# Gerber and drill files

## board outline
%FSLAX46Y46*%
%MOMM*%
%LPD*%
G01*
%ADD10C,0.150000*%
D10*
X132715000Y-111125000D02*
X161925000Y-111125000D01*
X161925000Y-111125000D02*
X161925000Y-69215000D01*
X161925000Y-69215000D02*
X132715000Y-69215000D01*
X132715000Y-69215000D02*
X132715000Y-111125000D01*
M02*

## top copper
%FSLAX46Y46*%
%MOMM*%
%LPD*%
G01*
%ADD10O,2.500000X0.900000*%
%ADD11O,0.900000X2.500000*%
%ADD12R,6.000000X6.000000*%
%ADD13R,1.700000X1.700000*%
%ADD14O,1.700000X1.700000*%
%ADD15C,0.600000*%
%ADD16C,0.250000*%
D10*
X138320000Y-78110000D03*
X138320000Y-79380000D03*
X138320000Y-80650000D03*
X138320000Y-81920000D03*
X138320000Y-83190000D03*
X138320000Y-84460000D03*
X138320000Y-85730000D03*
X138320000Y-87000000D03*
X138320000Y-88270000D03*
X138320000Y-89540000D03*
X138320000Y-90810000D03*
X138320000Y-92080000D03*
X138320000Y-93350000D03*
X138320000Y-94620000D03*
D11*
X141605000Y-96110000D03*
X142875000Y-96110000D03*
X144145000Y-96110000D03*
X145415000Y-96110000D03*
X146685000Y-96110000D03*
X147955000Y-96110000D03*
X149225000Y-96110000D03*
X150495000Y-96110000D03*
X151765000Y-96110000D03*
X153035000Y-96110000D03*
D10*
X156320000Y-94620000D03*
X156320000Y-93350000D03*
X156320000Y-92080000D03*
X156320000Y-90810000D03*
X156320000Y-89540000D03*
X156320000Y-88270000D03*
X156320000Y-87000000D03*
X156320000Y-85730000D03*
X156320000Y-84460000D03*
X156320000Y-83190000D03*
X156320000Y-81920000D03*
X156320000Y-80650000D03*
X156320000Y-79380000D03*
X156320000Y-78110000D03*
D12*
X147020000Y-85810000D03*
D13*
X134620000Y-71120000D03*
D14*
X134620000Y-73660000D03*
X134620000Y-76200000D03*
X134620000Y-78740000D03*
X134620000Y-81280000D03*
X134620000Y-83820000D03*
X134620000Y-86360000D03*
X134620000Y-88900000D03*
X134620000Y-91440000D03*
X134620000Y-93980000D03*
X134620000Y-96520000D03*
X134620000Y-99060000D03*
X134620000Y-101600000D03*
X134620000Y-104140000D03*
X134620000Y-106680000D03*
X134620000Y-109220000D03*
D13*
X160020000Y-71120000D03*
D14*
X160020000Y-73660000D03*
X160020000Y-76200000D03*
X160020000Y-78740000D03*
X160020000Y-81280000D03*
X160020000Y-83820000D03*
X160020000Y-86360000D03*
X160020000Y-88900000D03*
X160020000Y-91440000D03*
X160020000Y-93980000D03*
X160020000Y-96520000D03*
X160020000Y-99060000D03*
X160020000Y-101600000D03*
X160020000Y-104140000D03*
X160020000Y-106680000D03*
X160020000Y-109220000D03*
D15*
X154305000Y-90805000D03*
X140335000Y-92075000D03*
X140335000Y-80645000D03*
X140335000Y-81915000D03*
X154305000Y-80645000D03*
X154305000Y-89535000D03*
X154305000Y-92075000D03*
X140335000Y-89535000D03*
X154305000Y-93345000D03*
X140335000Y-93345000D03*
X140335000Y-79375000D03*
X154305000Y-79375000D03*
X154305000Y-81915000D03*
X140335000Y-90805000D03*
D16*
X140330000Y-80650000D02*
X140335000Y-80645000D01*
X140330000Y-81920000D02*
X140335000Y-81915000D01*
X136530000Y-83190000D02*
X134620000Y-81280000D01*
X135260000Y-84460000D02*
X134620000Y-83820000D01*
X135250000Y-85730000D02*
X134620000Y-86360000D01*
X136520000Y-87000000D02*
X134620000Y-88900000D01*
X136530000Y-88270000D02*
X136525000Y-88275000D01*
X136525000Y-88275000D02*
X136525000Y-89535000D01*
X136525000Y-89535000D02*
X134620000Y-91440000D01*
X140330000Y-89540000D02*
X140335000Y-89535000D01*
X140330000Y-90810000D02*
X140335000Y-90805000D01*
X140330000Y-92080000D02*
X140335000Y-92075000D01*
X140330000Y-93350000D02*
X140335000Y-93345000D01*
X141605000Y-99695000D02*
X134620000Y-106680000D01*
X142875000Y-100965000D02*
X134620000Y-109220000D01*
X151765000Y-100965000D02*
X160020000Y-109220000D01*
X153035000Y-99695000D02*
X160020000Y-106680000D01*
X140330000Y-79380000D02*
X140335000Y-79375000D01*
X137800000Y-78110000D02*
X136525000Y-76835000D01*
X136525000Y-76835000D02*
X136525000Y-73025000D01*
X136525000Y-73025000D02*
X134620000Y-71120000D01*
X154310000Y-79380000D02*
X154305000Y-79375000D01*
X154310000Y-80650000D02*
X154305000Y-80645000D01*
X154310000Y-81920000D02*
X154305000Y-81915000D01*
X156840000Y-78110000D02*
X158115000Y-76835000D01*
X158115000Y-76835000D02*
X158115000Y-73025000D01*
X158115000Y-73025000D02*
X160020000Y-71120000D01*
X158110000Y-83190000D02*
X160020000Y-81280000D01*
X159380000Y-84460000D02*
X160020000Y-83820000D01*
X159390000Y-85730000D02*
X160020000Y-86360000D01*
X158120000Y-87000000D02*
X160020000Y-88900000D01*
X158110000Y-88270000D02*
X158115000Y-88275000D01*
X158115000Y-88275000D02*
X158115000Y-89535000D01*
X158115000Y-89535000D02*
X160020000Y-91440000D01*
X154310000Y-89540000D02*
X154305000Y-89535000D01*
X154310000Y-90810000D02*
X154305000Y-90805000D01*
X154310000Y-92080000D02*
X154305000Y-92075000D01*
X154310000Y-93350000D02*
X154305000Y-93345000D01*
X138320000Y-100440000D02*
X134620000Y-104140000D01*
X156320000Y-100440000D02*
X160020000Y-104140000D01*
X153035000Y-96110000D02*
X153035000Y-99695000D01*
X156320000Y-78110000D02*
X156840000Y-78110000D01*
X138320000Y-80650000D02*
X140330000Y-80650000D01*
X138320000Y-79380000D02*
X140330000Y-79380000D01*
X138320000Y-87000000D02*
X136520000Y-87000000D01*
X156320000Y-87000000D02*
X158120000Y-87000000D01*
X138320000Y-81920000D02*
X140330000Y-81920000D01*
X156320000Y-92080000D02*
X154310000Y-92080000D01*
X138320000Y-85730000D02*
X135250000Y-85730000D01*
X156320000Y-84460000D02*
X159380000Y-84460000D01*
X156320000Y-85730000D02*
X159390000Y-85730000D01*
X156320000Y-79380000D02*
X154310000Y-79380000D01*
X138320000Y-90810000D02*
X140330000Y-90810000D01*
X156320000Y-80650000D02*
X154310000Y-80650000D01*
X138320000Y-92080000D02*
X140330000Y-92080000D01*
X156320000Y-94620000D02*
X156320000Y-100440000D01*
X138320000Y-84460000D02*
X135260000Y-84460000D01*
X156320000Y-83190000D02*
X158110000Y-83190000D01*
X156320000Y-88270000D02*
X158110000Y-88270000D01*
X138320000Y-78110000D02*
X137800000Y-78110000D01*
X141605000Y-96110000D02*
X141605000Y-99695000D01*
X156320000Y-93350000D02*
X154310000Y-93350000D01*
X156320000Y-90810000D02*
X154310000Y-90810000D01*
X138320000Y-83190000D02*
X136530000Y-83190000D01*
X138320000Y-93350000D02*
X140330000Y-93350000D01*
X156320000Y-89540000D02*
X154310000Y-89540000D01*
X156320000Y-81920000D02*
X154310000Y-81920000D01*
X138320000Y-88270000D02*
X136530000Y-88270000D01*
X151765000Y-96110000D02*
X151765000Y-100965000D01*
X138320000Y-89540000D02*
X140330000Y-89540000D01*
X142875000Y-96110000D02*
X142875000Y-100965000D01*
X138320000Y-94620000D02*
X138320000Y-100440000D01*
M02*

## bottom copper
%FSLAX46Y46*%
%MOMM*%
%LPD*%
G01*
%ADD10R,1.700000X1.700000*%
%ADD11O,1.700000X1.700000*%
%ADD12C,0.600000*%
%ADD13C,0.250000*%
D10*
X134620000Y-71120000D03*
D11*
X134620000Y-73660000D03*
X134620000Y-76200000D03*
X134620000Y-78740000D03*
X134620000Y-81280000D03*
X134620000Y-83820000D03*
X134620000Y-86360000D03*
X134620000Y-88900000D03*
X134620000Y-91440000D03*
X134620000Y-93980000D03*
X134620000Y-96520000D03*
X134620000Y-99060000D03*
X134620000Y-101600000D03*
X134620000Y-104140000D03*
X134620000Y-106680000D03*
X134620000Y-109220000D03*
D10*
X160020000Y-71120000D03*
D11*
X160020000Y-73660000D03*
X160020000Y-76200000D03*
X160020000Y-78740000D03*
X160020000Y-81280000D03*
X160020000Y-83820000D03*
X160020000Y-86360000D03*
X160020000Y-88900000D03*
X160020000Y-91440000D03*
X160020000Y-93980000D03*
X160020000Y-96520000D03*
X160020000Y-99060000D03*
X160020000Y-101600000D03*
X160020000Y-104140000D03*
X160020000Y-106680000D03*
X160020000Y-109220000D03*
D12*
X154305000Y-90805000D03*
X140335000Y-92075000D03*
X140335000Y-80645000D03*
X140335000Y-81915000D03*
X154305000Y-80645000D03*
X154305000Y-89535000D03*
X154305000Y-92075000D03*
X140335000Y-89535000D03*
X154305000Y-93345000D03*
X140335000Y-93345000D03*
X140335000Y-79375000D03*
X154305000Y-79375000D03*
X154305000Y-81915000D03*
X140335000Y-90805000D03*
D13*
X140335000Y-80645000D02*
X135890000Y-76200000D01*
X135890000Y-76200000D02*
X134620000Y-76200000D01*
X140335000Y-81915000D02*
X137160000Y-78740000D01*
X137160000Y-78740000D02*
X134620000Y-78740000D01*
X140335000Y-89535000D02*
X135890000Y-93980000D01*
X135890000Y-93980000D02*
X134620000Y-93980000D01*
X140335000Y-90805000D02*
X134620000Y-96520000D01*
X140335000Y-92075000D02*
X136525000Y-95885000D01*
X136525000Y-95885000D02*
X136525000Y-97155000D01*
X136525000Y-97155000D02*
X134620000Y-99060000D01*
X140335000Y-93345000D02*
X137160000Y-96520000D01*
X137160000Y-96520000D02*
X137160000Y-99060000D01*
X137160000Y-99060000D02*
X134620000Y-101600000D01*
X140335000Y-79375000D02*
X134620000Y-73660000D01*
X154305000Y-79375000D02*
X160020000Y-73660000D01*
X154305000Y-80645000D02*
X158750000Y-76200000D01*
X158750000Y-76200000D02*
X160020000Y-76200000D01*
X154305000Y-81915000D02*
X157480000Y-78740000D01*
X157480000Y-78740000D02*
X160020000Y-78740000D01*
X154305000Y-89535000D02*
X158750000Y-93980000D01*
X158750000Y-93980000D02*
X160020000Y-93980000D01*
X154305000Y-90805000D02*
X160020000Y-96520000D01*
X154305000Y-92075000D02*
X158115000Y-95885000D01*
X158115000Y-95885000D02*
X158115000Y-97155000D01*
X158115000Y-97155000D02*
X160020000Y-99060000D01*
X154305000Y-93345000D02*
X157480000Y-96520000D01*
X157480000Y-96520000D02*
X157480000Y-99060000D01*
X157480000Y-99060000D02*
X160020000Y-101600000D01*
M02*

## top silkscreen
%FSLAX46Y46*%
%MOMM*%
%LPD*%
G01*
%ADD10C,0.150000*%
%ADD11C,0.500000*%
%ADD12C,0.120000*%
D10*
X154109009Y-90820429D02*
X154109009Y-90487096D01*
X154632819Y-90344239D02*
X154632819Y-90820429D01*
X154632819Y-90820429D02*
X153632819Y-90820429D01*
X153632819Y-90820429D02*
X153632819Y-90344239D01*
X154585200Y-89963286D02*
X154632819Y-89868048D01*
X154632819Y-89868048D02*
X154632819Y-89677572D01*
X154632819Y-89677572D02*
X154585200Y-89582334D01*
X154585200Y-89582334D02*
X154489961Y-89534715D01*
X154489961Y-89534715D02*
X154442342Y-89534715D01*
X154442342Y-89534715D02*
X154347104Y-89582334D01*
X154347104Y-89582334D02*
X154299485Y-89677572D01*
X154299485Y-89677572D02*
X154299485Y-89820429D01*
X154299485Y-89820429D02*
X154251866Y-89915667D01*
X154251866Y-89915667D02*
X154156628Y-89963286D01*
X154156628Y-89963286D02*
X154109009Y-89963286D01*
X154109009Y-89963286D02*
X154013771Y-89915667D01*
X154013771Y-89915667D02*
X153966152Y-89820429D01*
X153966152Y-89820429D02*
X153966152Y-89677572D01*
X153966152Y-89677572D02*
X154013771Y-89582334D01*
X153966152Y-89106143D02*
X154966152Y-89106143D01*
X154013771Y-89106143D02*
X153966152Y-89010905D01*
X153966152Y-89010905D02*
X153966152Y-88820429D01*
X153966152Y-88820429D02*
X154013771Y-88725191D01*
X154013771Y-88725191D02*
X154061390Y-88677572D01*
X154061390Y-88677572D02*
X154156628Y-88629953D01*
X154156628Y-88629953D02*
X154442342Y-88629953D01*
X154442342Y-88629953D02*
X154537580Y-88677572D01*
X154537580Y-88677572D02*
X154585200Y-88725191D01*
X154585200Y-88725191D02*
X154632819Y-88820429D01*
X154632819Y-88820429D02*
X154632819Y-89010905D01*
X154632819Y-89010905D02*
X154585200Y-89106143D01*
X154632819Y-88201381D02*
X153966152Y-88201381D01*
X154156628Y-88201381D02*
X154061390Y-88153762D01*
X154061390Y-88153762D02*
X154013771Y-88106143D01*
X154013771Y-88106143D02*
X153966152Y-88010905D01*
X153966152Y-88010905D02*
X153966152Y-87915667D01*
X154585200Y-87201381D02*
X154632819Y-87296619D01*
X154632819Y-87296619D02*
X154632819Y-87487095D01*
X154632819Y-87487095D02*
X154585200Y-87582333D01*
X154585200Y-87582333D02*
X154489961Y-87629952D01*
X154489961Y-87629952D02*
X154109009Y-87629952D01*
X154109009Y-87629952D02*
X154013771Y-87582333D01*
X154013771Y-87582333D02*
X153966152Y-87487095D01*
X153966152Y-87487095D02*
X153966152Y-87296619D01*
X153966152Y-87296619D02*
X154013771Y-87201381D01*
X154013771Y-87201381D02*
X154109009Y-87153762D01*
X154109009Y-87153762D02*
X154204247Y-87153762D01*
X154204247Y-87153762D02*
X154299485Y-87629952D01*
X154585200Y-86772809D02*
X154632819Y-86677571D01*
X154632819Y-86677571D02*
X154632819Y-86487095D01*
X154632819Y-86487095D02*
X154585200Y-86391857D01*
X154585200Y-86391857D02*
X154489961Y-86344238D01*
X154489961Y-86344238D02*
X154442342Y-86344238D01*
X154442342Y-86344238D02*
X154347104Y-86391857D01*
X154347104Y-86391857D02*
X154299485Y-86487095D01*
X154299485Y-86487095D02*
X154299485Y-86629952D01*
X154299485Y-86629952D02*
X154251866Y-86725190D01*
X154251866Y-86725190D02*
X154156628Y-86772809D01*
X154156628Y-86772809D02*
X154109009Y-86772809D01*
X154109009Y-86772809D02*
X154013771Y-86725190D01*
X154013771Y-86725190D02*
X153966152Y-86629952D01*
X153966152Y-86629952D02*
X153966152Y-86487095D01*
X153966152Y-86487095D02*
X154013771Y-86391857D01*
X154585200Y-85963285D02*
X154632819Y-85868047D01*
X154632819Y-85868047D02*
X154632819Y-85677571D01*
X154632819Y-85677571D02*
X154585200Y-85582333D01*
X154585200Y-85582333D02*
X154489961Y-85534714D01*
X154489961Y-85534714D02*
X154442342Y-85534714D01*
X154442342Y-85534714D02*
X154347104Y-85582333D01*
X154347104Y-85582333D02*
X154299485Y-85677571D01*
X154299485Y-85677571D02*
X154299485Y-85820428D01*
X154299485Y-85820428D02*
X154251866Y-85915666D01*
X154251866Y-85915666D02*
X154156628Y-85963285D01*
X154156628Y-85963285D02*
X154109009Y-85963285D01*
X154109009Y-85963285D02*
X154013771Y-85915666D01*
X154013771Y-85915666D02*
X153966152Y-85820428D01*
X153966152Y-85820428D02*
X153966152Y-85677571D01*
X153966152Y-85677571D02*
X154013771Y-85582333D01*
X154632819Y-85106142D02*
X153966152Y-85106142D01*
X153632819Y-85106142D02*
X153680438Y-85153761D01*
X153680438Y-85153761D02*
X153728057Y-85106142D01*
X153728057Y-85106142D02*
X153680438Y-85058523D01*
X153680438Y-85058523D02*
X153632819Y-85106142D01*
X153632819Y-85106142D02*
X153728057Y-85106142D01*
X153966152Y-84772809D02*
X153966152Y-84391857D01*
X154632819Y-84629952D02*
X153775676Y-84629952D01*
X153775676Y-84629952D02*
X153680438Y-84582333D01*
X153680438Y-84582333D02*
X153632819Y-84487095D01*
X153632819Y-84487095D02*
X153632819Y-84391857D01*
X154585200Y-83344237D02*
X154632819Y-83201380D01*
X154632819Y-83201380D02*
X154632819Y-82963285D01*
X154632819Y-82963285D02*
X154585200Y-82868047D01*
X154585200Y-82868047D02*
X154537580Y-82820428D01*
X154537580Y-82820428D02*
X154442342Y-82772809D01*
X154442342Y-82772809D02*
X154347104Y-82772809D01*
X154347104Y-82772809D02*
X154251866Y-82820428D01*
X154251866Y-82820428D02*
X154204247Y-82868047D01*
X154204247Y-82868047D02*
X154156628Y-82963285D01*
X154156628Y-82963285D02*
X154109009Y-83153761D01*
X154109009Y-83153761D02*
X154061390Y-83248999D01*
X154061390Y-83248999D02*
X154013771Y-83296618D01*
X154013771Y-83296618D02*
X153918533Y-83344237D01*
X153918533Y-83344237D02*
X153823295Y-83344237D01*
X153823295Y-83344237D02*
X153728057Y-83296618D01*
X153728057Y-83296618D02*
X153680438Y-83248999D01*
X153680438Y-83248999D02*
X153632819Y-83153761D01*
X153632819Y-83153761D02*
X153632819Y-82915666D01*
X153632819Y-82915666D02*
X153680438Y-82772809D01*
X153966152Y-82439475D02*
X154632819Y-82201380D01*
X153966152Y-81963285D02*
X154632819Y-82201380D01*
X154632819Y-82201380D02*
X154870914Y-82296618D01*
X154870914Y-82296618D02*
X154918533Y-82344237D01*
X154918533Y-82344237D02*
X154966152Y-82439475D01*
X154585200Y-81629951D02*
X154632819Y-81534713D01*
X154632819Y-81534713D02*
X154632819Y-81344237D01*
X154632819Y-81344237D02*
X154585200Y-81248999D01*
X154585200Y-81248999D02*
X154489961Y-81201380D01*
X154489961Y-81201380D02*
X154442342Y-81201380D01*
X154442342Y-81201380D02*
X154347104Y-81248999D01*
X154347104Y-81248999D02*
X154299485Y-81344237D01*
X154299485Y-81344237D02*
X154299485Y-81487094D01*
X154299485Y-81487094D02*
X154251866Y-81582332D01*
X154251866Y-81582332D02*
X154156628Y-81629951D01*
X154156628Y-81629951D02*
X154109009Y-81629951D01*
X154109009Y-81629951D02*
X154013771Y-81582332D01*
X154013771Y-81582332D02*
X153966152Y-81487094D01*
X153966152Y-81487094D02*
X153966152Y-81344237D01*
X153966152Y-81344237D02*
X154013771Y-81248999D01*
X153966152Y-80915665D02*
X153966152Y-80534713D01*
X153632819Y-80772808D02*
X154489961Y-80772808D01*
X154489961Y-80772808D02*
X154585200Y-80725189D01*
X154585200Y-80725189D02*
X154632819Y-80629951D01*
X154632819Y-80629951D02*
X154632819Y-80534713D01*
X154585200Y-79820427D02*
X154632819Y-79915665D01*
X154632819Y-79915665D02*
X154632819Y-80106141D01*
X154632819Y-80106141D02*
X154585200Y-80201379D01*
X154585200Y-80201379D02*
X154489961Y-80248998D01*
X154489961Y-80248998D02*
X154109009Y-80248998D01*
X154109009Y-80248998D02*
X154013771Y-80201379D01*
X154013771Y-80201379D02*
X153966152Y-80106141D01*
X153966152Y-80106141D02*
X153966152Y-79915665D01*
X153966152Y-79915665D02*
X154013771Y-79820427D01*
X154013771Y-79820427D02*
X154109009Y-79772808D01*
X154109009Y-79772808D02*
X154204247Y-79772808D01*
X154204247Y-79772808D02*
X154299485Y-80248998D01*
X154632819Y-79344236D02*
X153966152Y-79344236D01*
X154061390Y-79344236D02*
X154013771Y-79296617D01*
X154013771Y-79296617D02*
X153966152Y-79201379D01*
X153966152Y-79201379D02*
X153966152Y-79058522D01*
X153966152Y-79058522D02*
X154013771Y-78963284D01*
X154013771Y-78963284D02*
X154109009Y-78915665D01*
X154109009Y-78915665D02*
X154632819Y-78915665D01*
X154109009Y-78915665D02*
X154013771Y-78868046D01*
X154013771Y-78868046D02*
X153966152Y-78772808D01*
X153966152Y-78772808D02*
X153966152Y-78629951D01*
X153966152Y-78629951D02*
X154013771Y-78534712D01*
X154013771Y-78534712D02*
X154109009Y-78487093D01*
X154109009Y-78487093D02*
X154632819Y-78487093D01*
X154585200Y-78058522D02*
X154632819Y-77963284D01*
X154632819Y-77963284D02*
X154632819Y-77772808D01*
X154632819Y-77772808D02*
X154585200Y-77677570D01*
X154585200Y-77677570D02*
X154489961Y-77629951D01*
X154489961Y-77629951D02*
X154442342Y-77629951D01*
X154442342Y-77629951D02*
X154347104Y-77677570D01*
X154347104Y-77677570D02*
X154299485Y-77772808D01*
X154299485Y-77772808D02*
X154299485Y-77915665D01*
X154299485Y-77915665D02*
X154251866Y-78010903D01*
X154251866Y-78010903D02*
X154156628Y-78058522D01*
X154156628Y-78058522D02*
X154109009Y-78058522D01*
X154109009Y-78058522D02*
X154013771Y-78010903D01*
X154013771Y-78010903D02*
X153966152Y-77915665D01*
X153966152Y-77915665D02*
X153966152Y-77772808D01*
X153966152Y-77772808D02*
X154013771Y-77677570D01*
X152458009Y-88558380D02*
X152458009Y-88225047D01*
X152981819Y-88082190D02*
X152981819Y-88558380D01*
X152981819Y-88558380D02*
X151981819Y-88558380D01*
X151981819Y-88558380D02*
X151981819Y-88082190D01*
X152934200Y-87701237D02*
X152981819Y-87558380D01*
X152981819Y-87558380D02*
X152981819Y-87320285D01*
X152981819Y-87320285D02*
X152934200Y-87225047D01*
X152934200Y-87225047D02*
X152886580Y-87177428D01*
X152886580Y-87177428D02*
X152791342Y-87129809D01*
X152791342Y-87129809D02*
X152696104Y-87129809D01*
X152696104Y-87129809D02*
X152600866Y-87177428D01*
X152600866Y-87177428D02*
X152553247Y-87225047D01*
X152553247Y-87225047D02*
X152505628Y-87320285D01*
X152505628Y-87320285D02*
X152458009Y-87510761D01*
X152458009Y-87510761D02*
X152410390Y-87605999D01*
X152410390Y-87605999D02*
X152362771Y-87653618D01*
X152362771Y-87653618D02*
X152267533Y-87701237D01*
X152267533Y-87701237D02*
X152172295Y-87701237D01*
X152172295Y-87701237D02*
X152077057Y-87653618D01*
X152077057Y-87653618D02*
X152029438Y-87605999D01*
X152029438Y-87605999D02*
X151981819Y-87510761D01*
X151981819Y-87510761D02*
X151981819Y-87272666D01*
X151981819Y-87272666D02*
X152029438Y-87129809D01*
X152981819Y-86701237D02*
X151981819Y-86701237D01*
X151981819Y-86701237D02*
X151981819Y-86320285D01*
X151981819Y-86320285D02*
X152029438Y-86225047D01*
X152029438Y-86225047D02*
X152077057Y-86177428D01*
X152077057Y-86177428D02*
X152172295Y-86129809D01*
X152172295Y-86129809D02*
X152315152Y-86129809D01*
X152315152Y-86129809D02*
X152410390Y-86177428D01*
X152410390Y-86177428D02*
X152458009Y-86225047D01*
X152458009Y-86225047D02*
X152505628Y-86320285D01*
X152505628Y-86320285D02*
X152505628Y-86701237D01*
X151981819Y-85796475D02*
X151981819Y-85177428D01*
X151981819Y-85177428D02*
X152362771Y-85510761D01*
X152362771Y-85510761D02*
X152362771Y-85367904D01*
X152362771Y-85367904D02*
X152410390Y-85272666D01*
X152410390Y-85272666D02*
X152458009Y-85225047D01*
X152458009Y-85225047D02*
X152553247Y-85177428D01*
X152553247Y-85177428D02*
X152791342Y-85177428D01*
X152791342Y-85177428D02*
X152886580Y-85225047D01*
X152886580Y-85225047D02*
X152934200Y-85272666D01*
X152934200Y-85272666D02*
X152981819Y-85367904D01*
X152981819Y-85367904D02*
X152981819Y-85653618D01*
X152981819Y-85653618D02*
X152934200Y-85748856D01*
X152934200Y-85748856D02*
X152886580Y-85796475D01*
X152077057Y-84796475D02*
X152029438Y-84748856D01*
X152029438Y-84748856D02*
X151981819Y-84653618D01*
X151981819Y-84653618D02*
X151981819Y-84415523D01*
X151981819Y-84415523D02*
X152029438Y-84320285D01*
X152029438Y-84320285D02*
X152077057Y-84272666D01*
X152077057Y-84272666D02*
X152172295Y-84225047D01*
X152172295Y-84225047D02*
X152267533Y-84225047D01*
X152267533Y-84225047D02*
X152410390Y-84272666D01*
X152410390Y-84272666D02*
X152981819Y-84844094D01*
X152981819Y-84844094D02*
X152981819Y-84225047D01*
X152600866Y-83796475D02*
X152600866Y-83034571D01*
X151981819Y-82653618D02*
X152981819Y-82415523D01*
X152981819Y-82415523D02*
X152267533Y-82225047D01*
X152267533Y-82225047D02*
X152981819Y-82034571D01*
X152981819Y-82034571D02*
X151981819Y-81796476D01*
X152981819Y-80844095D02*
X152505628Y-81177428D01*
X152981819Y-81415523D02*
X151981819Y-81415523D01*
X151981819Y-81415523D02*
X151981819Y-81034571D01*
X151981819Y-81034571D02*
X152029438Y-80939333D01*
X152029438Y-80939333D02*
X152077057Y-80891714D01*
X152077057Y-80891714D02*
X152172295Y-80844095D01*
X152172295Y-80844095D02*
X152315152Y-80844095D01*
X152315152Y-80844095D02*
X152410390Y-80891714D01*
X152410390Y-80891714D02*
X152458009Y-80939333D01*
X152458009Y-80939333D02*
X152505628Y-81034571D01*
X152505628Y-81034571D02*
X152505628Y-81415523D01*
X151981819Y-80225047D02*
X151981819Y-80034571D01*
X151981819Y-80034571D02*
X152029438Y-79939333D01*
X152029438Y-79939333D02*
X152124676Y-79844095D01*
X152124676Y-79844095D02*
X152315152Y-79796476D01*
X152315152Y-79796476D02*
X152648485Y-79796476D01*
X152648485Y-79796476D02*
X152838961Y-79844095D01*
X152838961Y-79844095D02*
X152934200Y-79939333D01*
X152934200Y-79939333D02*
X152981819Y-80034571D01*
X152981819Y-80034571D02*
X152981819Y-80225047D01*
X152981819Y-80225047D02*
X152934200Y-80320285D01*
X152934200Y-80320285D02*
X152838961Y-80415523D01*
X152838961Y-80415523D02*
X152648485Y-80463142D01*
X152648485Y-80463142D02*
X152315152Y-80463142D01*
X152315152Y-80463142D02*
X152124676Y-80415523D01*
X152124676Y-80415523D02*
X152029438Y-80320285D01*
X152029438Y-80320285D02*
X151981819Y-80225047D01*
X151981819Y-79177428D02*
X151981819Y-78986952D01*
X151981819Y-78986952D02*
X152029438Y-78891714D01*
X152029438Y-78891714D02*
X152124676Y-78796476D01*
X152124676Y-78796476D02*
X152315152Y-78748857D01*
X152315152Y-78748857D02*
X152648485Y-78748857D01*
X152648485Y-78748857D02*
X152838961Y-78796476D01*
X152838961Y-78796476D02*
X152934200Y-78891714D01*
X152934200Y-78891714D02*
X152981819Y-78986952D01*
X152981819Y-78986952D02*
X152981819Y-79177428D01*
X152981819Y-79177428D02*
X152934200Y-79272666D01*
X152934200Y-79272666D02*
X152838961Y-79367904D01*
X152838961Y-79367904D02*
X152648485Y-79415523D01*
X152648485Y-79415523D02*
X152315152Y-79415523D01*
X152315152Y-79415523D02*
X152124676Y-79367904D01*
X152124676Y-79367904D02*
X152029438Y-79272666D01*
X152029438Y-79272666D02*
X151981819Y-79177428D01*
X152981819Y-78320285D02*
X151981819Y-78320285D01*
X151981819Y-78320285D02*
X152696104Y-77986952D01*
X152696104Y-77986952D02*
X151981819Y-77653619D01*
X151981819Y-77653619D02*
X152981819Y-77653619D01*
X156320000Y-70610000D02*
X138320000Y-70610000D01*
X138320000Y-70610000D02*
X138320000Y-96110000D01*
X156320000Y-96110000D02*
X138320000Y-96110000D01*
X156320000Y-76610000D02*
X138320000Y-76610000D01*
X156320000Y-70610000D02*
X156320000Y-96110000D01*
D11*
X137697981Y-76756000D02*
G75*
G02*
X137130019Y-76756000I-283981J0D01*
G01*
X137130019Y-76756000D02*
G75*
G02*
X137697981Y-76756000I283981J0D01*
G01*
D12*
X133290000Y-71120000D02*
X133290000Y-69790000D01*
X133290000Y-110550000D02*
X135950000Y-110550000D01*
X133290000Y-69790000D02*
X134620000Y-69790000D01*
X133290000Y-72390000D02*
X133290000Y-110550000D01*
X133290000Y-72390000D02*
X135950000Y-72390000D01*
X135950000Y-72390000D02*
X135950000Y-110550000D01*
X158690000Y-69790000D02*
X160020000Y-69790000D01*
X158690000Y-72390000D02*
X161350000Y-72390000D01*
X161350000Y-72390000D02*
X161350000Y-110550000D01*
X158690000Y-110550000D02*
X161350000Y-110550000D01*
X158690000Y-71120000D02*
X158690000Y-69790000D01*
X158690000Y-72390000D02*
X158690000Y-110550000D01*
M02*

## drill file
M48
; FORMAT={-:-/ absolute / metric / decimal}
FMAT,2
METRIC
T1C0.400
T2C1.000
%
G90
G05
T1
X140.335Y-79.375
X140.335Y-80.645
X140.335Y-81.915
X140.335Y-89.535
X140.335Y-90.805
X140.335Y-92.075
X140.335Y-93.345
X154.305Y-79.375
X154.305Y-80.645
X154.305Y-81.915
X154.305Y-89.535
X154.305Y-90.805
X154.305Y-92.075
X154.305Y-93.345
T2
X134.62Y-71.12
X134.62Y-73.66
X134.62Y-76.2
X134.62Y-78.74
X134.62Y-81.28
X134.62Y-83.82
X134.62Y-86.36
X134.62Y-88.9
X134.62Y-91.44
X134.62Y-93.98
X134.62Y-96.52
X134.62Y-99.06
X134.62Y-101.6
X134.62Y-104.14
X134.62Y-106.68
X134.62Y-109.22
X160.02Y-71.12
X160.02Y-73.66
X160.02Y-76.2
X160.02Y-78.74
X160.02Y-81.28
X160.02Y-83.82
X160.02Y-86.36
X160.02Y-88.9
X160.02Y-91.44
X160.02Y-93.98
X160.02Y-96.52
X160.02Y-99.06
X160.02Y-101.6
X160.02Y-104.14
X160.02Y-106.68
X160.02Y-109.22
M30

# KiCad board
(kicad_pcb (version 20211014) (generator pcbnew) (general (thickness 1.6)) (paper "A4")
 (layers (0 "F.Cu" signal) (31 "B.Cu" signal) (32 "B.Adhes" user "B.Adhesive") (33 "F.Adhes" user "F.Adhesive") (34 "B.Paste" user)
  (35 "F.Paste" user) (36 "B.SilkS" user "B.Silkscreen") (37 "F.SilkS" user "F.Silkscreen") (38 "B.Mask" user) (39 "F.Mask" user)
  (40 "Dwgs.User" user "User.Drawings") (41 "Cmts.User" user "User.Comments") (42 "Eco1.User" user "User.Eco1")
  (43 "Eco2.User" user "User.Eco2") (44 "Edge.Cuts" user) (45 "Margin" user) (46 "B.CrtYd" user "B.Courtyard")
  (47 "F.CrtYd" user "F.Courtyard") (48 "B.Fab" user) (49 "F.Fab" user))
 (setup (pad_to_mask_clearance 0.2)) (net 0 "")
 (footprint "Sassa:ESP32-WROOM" (layer "F.Cu") (at 147.32 86.36 180)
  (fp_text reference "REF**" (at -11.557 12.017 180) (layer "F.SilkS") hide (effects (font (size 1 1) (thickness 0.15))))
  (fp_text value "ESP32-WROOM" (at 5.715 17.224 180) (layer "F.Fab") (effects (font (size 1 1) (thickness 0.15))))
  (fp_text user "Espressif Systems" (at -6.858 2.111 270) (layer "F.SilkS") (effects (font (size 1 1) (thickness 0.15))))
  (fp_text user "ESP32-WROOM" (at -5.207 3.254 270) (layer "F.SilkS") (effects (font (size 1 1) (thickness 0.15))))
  (fp_line (start -9 15.75) (end 9 15.75) (layer "F.SilkS") (width 0.15))
  (fp_line (start 9 15.75) (end 9 -9.75) (layer "F.SilkS") (width 0.15))
  (fp_line (start -9 -9.75) (end 9 -9.75) (layer "F.SilkS") (width 0.15))
  (fp_line (start -9 9.75) (end 9 9.75) (layer "F.SilkS") (width 0.15))
  (fp_line (start -9 15.75) (end -9 -9.75) (layer "F.SilkS") (width 0.15))
  (fp_circle (center 9.906 9.604) (end 10.033 9.858) (layer "F.SilkS") (width 0.5) (fill none))
  (pad "1" smd oval locked (at 9 8.25 180) (size 2.5 0.9) (layers "F.Cu" "F.Paste" "F.Mask"))
  (pad "2" smd oval locked (at 9 6.98 180) (size 2.5 0.9) (layers "F.Cu" "F.Paste" "F.Mask"))
  (pad "3" smd oval locked (at 9 5.71 180) (size 2.5 0.9) (layers "F.Cu" "F.Paste" "F.Mask"))
  (pad "4" smd oval locked (at 9 4.44 180) (size 2.5 0.9) (layers "F.Cu" "F.Paste" "F.Mask"))
  (pad "5" smd oval locked (at 9 3.17 180) (size 2.5 0.9) (layers "F.Cu" "F.Paste" "F.Mask"))
  (pad "6" smd oval locked (at 9 1.9 180) (size 2.5 0.9) (layers "F.Cu" "F.Paste" "F.Mask"))
  (pad "7" smd oval locked (at 9 0.63 180) (size 2.5 0.9) (layers "F.Cu" "F.Paste" "F.Mask"))
  (pad "8" smd oval locked (at 9 -0.64 180) (size 2.5 0.9) (layers "F.Cu" "F.Paste" "F.Mask"))
  (pad "9" smd oval locked (at 9 -1.91 180) (size 2.5 0.9) (layers "F.Cu" "F.Paste" "F.Mask"))
  (pad "10" smd oval locked (at 9 -3.18 180) (size 2.5 0.9) (layers "F.Cu" "F.Paste" "F.Mask"))
  (pad "11" smd oval locked (at 9 -4.45 180) (size 2.5 0.9) (layers "F.Cu" "F.Paste" "F.Mask"))
  (pad "12" smd oval locked (at 9 -5.72 180) (size 2.5 0.9) (layers "F.Cu" "F.Paste" "F.Mask"))
  (pad "13" smd oval locked (at 9 -6.99 180) (size 2.5 0.9) (layers "F.Cu" "F.Paste" "F.Mask"))
  (pad "14" smd oval locked (at 9 -8.26 180) (size 2.5 0.9) (layers "F.Cu" "F.Paste" "F.Mask"))
  (pad "15" smd oval locked (at 5.715 -9.75 180) (size 0.9 2.5) (layers "F.Cu" "F.Paste" "F.Mask"))
  (pad "16" smd oval locked (at 4.445 -9.75 180) (size 0.9 2.5) (layers "F.Cu" "F.Paste" "F.Mask"))
  (pad "17" smd oval locked (at 3.175 -9.75 180) (size 0.9 2.5) (layers "F.Cu" "F.Paste" "F.Mask"))
  (pad "18" smd oval locked (at 1.905 -9.75 180) (size 0.9 2.5) (layers "F.Cu" "F.Paste" "F.Mask"))
  (pad "19" smd oval locked (at 0.635 -9.75 180) (size 0.9 2.5) (layers "F.Cu" "F.Paste" "F.Mask"))
  (pad "20" smd oval locked (at -0.635 -9.75 180) (size 0.9 2.5) (layers "F.Cu" "F.Paste" "F.Mask"))
  (pad "21" smd oval locked (at -1.905 -9.75 180) (size 0.9 2.5) (layers "F.Cu" "F.Paste" "F.Mask"))
  (pad "22" smd oval locked (at -3.175 -9.75 180) (size 0.9 2.5) (layers "F.Cu" "F.Paste" "F.Mask"))
  (pad "23" smd oval locked (at -4.445 -9.75 180) (size 0.9 2.5) (layers "F.Cu" "F.Paste" "F.Mask"))
  (pad "24" smd oval locked (at -5.715 -9.75 180) (size 0.9 2.5) (layers "F.Cu" "F.Paste" "F.Mask"))
  (pad "25" smd oval locked (at -9 -8.26 180) (size 2.5 0.9) (layers "F.Cu" "F.Paste" "F.Mask"))
  (pad "26" smd oval locked (at -9 -6.99 180) (size 2.5 0.9) (layers "F.Cu" "F.Paste" "F.Mask"))
  (pad "27" smd oval locked (at -9 -5.72 180) (size 2.5 0.9) (layers "F.Cu" "F.Paste" "F.Mask"))
  (pad "28" smd oval locked (at -9 -4.45 180) (size 2.5 0.9) (layers "F.Cu" "F.Paste" "F.Mask"))
  (pad "29" smd oval locked (at -9 -3.18 180) (size 2.5 0.9) (layers "F.Cu" "F.Paste" "F.Mask"))
  (pad "30" smd oval locked (at -9 -1.91 180) (size 2.5 0.9) (layers "F.Cu" "F.Paste" "F.Mask"))
  (pad "31" smd oval locked (at -9 -0.64 180) (size 2.5 0.9) (layers "F.Cu" "F.Paste" "F.Mask"))
  (pad "32" smd oval locked (at -9 0.63 180) (size 2.5 0.9) (layers "F.Cu" "F.Paste" "F.Mask"))
  (pad "33" smd oval locked (at -9 1.9 180) (size 2.5 0.9) (layers "F.Cu" "F.Paste" "F.Mask"))
  (pad "34" smd oval locked (at -9 3.17 180) (size 2.5 0.9) (layers "F.Cu" "F.Paste" "F.Mask"))
  (pad "35" smd oval locked (at -9 4.44 180) (size 2.5 0.9) (layers "F.Cu" "F.Paste" "F.Mask"))
  (pad "36" smd oval locked (at -9 5.71 180) (size 2.5 0.9) (layers "F.Cu" "F.Paste" "F.Mask"))
  (pad "37" smd oval locked (at -9 6.98 180) (size 2.5 0.9) (layers "F.Cu" "F.Paste" "F.Mask"))
  (pad "38" smd oval locked (at -9 8.25 180) (size 2.5 0.9) (layers "F.Cu" "F.Paste" "F.Mask"))
  (pad "39" smd rect locked (at 0.3 0.55 180) (size 6 6) (layers "F.Cu" "F.Paste" "F.Mask")))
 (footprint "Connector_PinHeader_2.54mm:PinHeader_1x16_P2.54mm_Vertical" (layer "F.Cu") (at 134.62 71.12)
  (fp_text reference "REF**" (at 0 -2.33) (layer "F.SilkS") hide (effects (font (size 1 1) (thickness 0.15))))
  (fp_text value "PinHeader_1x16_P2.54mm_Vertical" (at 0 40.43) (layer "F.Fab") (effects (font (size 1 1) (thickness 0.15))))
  (fp_line (start -1.33 0) (end -1.33 -1.33) (layer "F.SilkS") (width 0.12))
  (fp_line (start -1.33 39.43) (end 1.33 39.43) (layer "F.SilkS") (width 0.12))
  (fp_line (start -1.33 -1.33) (end 0 -1.33) (layer "F.SilkS") (width 0.12))
  (fp_line (start -1.33 1.27) (end -1.33 39.43) (layer "F.SilkS") (width 0.12))
  (fp_line (start -1.33 1.27) (end 1.33 1.27) (layer "F.SilkS") (width 0.12))
  (fp_line (start 1.33 1.27) (end 1.33 39.43) (layer "F.SilkS") (width 0.12))
  (pad "1" thru_hole rect (at 0 0) (size 1.7 1.7) (drill 1) (layers *.Cu *.Mask))
  (pad "2" thru_hole oval (at 0 2.54) (size 1.7 1.7) (drill 1) (layers *.Cu *.Mask))
  (pad "3" thru_hole oval (at 0 5.08) (size 1.7 1.7) (drill 1) (layers *.Cu *.Mask))
  (pad "4" thru_hole oval (at 0 7.62) (size 1.7 1.7) (drill 1) (layers *.Cu *.Mask))
  (pad "5" thru_hole oval (at 0 10.16) (size 1.7 1.7) (drill 1) (layers *.Cu *.Mask))
  (pad "6" thru_hole oval (at 0 12.7) (size 1.7 1.7) (drill 1) (layers *.Cu *.Mask))
  (pad "7" thru_hole oval (at 0 15.24) (size 1.7 1.7) (drill 1) (layers *.Cu *.Mask))
  (pad "8" thru_hole oval (at 0 17.78) (size 1.7 1.7) (drill 1) (layers *.Cu *.Mask))
  (pad "9" thru_hole oval (at 0 20.32) (size 1.7 1.7) (drill 1) (layers *.Cu *.Mask))
  (pad "10" thru_hole oval (at 0 22.86) (size 1.7 1.7) (drill 1) (layers *.Cu *.Mask))
  (pad "11" thru_hole oval (at 0 25.4) (size 1.7 1.7) (drill 1) (layers *.Cu *.Mask))
  (pad "12" thru_hole oval (at 0 27.94) (size 1.7 1.7) (drill 1) (layers *.Cu *.Mask))
  (pad "13" thru_hole oval (at 0 30.48) (size 1.7 1.7) (drill 1) (layers *.Cu *.Mask))
  (pad "14" thru_hole oval (at 0 33.02) (size 1.7 1.7) (drill 1) (layers *.Cu *.Mask))
  (pad "15" thru_hole oval (at 0 35.56) (size 1.7 1.7) (drill 1) (layers *.Cu *.Mask))
  (pad "16" thru_hole oval (at 0 38.1) (size 1.7 1.7) (drill 1) (layers *.Cu *.Mask)))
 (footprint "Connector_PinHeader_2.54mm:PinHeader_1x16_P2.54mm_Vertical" (layer "F.Cu") (at 160.02 71.12)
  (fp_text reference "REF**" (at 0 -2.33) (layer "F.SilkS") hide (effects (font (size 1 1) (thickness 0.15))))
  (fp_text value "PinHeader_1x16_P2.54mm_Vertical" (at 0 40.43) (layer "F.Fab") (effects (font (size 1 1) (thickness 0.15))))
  (fp_line (start -1.33 -1.33) (end 0 -1.33) (layer "F.SilkS") (width 0.12))
  (fp_line (start -1.33 1.27) (end 1.33 1.27) (layer "F.SilkS") (width 0.12))
  (fp_line (start 1.33 1.27) (end 1.33 39.43) (layer "F.SilkS") (width 0.12))
  (fp_line (start -1.33 39.43) (end 1.33 39.43) (layer "F.SilkS") (width 0.12))
  (fp_line (start -1.33 0) (end -1.33 -1.33) (layer "F.SilkS") (width 0.12))
  (fp_line (start -1.33 1.27) (end -1.33 39.43) (layer "F.SilkS") (width 0.12))
  (pad "1" thru_hole rect (at 0 0) (size 1.7 1.7) (drill 1) (layers *.Cu *.Mask))
  (pad "2" thru_hole oval (at 0 2.54) (size 1.7 1.7) (drill 1) (layers *.Cu *.Mask))
  (pad "3" thru_hole oval (at 0 5.08) (size 1.7 1.7) (drill 1) (layers *.Cu *.Mask))
  (pad "4" thru_hole oval (at 0 7.62) (size 1.7 1.7) (drill 1) (layers *.Cu *.Mask))
  (pad "5" thru_hole oval (at 0 10.16) (size 1.7 1.7) (drill 1) (layers *.Cu *.Mask))
  (pad "6" thru_hole oval (at 0 12.7) (size 1.7 1.7) (drill 1) (layers *.Cu *.Mask))
  (pad "7" thru_hole oval (at 0 15.24) (size 1.7 1.7) (drill 1) (layers *.Cu *.Mask))
  (pad "8" thru_hole oval (at 0 17.78) (size 1.7 1.7) (drill 1) (layers *.Cu *.Mask))
  (pad "9" thru_hole oval (at 0 20.32) (size 1.7 1.7) (drill 1) (layers *.Cu *.Mask))
  (pad "10" thru_hole oval (at 0 22.86) (size 1.7 1.7) (drill 1) (layers *.Cu *.Mask))
  (pad "11" thru_hole oval (at 0 25.4) (size 1.7 1.7) (drill 1) (layers *.Cu *.Mask))
  (pad "12" thru_hole oval (at 0 27.94) (size 1.7 1.7) (drill 1) (layers *.Cu *.Mask))
  (pad "13" thru_hole oval (at 0 30.48) (size 1.7 1.7) (drill 1) (layers *.Cu *.Mask))
  (pad "14" thru_hole oval (at 0 33.02) (size 1.7 1.7) (drill 1) (layers *.Cu *.Mask))
  (pad "15" thru_hole oval (at 0 35.56) (size 1.7 1.7) (drill 1) (layers *.Cu *.Mask))
  (pad "16" thru_hole oval (at 0 38.1) (size 1.7 1.7) (drill 1) (layers *.Cu *.Mask)))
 (gr_line (start 132.715 111.125) (end 161.925 111.125) (layer "Edge.Cuts") (width 0.15))
 (gr_line (start 161.925 111.125) (end 161.925 69.215) (layer "Edge.Cuts") (width 0.15))
 (gr_line (start 161.925 69.215) (end 132.715 69.215) (layer "Edge.Cuts") (width 0.15))
 (gr_line (start 132.715 69.215) (end 132.715 111.125) (layer "Edge.Cuts") (width 0.15))
 (segment (start 140.33 80.65) (end 140.335 80.645) (width 0.25) (layer "F.Cu") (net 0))
 (segment (start 140.33 81.92) (end 140.335 81.915) (width 0.25) (layer "F.Cu") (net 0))
 (segment (start 136.53 83.19) (end 134.62 81.28) (width 0.25) (layer "F.Cu") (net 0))
 (segment (start 135.26 84.46) (end 134.62 83.82) (width 0.25) (layer "F.Cu") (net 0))
 (segment (start 135.25 85.73) (end 134.62 86.36) (width 0.25) (layer "F.Cu") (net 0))
 (segment (start 136.52 87) (end 134.62 88.9) (width 0.25) (layer "F.Cu") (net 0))
 (segment (start 136.53 88.27) (end 136.525 88.275) (width 0.25) (layer "F.Cu") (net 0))
 (segment (start 136.525 88.275) (end 136.525 89.535) (width 0.25) (layer "F.Cu") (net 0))
 (segment (start 136.525 89.535) (end 134.62 91.44) (width 0.25) (layer "F.Cu") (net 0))
 (segment (start 140.33 89.54) (end 140.335 89.535) (width 0.25) (layer "F.Cu") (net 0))
 (segment (start 140.33 90.81) (end 140.335 90.805) (width 0.25) (layer "F.Cu") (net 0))
 (segment (start 140.33 92.08) (end 140.335 92.075) (width 0.25) (layer "F.Cu") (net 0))
 (segment (start 140.33 93.35) (end 140.335 93.345) (width 0.25) (layer "F.Cu") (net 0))
 (segment (start 141.605 99.695) (end 134.62 106.68) (width 0.25) (layer "F.Cu") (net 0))
 (segment (start 142.875 100.965) (end 134.62 109.22) (width 0.25) (layer "F.Cu") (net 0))
 (segment (start 151.765 100.965) (end 160.02 109.22) (width 0.25) (layer "F.Cu") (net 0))
 (segment (start 153.035 99.695) (end 160.02 106.68) (width 0.25) (layer "F.Cu") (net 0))
 (segment (start 140.33 79.38) (end 140.335 79.375) (width 0.25) (layer "F.Cu") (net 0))
 (segment (start 137.8 78.11) (end 136.525 76.835) (width 0.25) (layer "F.Cu") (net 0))
 (segment (start 136.525 76.835) (end 136.525 73.025) (width 0.25) (layer "F.Cu") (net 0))
 (segment (start 136.525 73.025) (end 134.62 71.12) (width 0.25) (layer "F.Cu") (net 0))
 (segment (start 154.31 79.38) (end 154.305 79.375) (width 0.25) (layer "F.Cu") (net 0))
 (segment (start 154.31 80.65) (end 154.305 80.645) (width 0.25) (layer "F.Cu") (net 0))
 (segment (start 154.31 81.92) (end 154.305 81.915) (width 0.25) (layer "F.Cu") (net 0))
 (segment (start 156.84 78.11) (end 158.115 76.835) (width 0.25) (layer "F.Cu") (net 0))
 (segment (start 158.115 76.835) (end 158.115 73.025) (width 0.25) (layer "F.Cu") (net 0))
 (segment (start 158.115 73.025) (end 160.02 71.12) (width 0.25) (layer "F.Cu") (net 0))
 (segment (start 158.11 83.19) (end 160.02 81.28) (width 0.25) (layer "F.Cu") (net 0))
 (segment (start 159.38 84.46) (end 160.02 83.82) (width 0.25) (layer "F.Cu") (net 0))
 (segment (start 159.39 85.73) (end 160.02 86.36) (width 0.25) (layer "F.Cu") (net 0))
 (segment (start 158.12 87) (end 160.02 88.9) (width 0.25) (layer "F.Cu") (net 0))
 (segment (start 158.11 88.27) (end 158.115 88.275) (width 0.25) (layer "F.Cu") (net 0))
 (segment (start 158.115 88.275) (end 158.115 89.535) (width 0.25) (layer "F.Cu") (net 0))
 (segment (start 158.115 89.535) (end 160.02 91.44) (width 0.25) (layer "F.Cu") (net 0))
 (segment (start 154.31 89.54) (end 154.305 89.535) (width 0.25) (layer "F.Cu") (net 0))
 (segment (start 154.31 90.81) (end 154.305 90.805) (width 0.25) (layer "F.Cu") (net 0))
 (segment (start 154.31 92.08) (end 154.305 92.075) (width 0.25) (layer "F.Cu") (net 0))
 (segment (start 154.31 93.35) (end 154.305 93.345) (width 0.25) (layer "F.Cu") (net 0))
 (segment (start 138.32 100.44) (end 134.62 104.14) (width 0.25) (layer "F.Cu") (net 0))
 (segment (start 156.32 100.44) (end 160.02 104.14) (width 0.25) (layer "F.Cu") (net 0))
 (segment (start 153.035 96.11) (end 153.035 99.695) (width 0.25) (layer "F.Cu") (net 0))
 (segment (start 156.32 78.11) (end 156.84 78.11) (width 0.25) (layer "F.Cu") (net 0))
 (segment (start 138.32 80.65) (end 140.33 80.65) (width 0.25) (layer "F.Cu") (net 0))
 (segment (start 138.32 79.38) (end 140.33 79.38) (width 0.25) (layer "F.Cu") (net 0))
 (segment (start 138.32 87) (end 136.52 87) (width 0.25) (layer "F.Cu") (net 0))
 (segment (start 156.32 87) (end 158.12 87) (width 0.25) (layer "F.Cu") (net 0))
 (segment (start 138.32 81.92) (end 140.33 81.92) (width 0.25) (layer "F.Cu") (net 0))
 (segment (start 156.32 92.08) (end 154.31 92.08) (width 0.25) (layer "F.Cu") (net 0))
 (segment (start 138.32 85.73) (end 135.25 85.73) (width 0.25) (layer "F.Cu") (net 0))
 (segment (start 156.32 84.46) (end 159.38 84.46) (width 0.25) (layer "F.Cu") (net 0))
 (segment (start 156.32 85.73) (end 159.39 85.73) (width 0.25) (layer "F.Cu") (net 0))
 (segment (start 156.32 79.38) (end 154.31 79.38) (width 0.25) (layer "F.Cu") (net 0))
 (segment (start 138.32 90.81) (end 140.33 90.81) (width 0.25) (layer "F.Cu") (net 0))
 (segment (start 156.32 80.65) (end 154.31 80.65) (width 0.25) (layer "F.Cu") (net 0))
 (segment (start 138.32 92.08) (end 140.33 92.08) (width 0.25) (layer "F.Cu") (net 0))
 (segment (start 156.32 94.62) (end 156.32 100.44) (width 0.25) (layer "F.Cu") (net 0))
 (segment (start 138.32 84.46) (end 135.26 84.46) (width 0.25) (layer "F.Cu") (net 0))
 (segment (start 156.32 83.19) (end 158.11 83.19) (width 0.25) (layer "F.Cu") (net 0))
 (segment (start 156.32 88.27) (end 158.11 88.27) (width 0.25) (layer "F.Cu") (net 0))
 (segment (start 138.32 78.11) (end 137.8 78.11) (width 0.25) (layer "F.Cu") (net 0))
 (segment (start 141.605 96.11) (end 141.605 99.695) (width 0.25) (layer "F.Cu") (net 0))
 (segment (start 156.32 93.35) (end 154.31 93.35) (width 0.25) (layer "F.Cu") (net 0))
 (segment (start 156.32 90.81) (end 154.31 90.81) (width 0.25) (layer "F.Cu") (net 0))
 (segment (start 138.32 83.19) (end 136.53 83.19) (width 0.25) (layer "F.Cu") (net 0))
 (segment (start 138.32 93.35) (end 140.33 93.35) (width 0.25) (layer "F.Cu") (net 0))
 (segment (start 156.32 89.54) (end 154.31 89.54) (width 0.25) (layer "F.Cu") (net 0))
 (segment (start 156.32 81.92) (end 154.31 81.92) (width 0.25) (layer "F.Cu") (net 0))
 (segment (start 138.32 88.27) (end 136.53 88.27) (width 0.25) (layer "F.Cu") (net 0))
 (segment (start 151.765 96.11) (end 151.765 100.965) (width 0.25) (layer "F.Cu") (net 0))
 (segment (start 138.32 89.54) (end 140.33 89.54) (width 0.25) (layer "F.Cu") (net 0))
 (segment (start 142.875 96.11) (end 142.875 100.965) (width 0.25) (layer "F.Cu") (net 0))
 (segment (start 138.32 94.62) (end 138.32 100.44) (width 0.25) (layer "F.Cu") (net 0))
 (via (at 154.305 90.805) (size 0.6) (drill 0.4) (layers "F.Cu" "B.Cu") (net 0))
 (via (at 140.335 92.075) (size 0.6) (drill 0.4) (layers "F.Cu" "B.Cu") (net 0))
 (via (at 140.335 80.645) (size 0.6) (drill 0.4) (layers "F.Cu" "B.Cu") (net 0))
 (via (at 140.335 81.915) (size 0.6) (drill 0.4) (layers "F.Cu" "B.Cu") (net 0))
 (via (at 154.305 80.645) (size 0.6) (drill 0.4) (layers "F.Cu" "B.Cu") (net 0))
 (via (at 154.305 89.535) (size 0.6) (drill 0.4) (layers "F.Cu" "B.Cu") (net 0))
 (via (at 154.305 92.075) (size 0.6) (drill 0.4) (layers "F.Cu" "B.Cu") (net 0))
 (via (at 140.335 89.535) (size 0.6) (drill 0.4) (layers "F.Cu" "B.Cu") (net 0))
 (via (at 154.305 93.345) (size 0.6) (drill 0.4) (layers "F.Cu" "B.Cu") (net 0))
 (via (at 140.335 93.345) (size 0.6) (drill 0.4) (layers "F.Cu" "B.Cu") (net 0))
 (via (at 140.335 79.375) (size 0.6) (drill 0.4) (layers "F.Cu" "B.Cu") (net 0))
 (via (at 154.305 79.375) (size 0.6) (drill 0.4) (layers "F.Cu" "B.Cu") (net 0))
 (via (at 154.305 81.915) (size 0.6) (drill 0.4) (layers "F.Cu" "B.Cu") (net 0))
 (via (at 140.335 90.805) (size 0.6) (drill 0.4) (layers "F.Cu" "B.Cu") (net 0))
 (segment (start 140.335 80.645) (end 135.89 76.2) (width 0.25) (layer "B.Cu") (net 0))
 (segment (start 135.89 76.2) (end 134.62 76.2) (width 0.25) (layer "B.Cu") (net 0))
 (segment (start 140.335 81.915) (end 137.16 78.74) (width 0.25) (layer "B.Cu") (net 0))
 (segment (start 137.16 78.74) (end 134.62 78.74) (width 0.25) (layer "B.Cu") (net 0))
 (segment (start 140.335 89.535) (end 135.89 93.98) (width 0.25) (layer "B.Cu") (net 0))
 (segment (start 135.89 93.98) (end 134.62 93.98) (width 0.25) (layer "B.Cu") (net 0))
 (segment (start 140.335 90.805) (end 134.62 96.52) (width 0.25) (layer "B.Cu") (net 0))
 (segment (start 140.335 92.075) (end 136.525 95.885) (width 0.25) (layer "B.Cu") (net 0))
 (segment (start 136.525 95.885) (end 136.525 97.155) (width 0.25) (layer "B.Cu") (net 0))
 (segment (start 136.525 97.155) (end 134.62 99.06) (width 0.25) (layer "B.Cu") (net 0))
 (segment (start 140.335 93.345) (end 137.16 96.52) (width 0.25) (layer "B.Cu") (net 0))
 (segment (start 137.16 96.52) (end 137.16 99.06) (width 0.25) (layer "B.Cu") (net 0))
 (segment (start 137.16 99.06) (end 134.62 101.6) (width 0.25) (layer "B.Cu") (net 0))
 (segment (start 140.335 79.375) (end 134.62 73.66) (width 0.25) (layer "B.Cu") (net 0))
 (segment (start 154.305 79.375) (end 160.02 73.66) (width 0.25) (layer "B.Cu") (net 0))
 (segment (start 154.305 80.645) (end 158.75 76.2) (width 0.25) (layer "B.Cu") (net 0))
 (segment (start 158.75 76.2) (end 160.02 76.2) (width 0.25) (layer "B.Cu") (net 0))
 (segment (start 154.305 81.915) (end 157.48 78.74) (width 0.25) (layer "B.Cu") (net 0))
 (segment (start 157.48 78.74) (end 160.02 78.74) (width 0.25) (layer "B.Cu") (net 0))
 (segment (start 154.305 89.535) (end 158.75 93.98) (width 0.25) (layer "B.Cu") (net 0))
 (segment (start 158.75 93.98) (end 160.02 93.98) (width 0.25) (layer "B.Cu") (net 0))
 (segment (start 154.305 90.805) (end 160.02 96.52) (width 0.25) (layer "B.Cu") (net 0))
 (segment (start 154.305 92.075) (end 158.115 95.885) (width 0.25) (layer "B.Cu") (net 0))
 (segment (start 158.115 95.885) (end 158.115 97.155) (width 0.25) (layer "B.Cu") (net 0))
 (segment (start 158.115 97.155) (end 160.02 99.06) (width 0.25) (layer "B.Cu") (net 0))
 (segment (start 154.305 93.345) (end 157.48 96.52) (width 0.25) (layer "B.Cu") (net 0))
 (segment (start 157.48 96.52) (end 157.48 99.06) (width 0.25) (layer "B.Cu") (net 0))
 (segment (start 157.48 99.06) (end 160.02 101.6) (width 0.25) (layer "B.Cu") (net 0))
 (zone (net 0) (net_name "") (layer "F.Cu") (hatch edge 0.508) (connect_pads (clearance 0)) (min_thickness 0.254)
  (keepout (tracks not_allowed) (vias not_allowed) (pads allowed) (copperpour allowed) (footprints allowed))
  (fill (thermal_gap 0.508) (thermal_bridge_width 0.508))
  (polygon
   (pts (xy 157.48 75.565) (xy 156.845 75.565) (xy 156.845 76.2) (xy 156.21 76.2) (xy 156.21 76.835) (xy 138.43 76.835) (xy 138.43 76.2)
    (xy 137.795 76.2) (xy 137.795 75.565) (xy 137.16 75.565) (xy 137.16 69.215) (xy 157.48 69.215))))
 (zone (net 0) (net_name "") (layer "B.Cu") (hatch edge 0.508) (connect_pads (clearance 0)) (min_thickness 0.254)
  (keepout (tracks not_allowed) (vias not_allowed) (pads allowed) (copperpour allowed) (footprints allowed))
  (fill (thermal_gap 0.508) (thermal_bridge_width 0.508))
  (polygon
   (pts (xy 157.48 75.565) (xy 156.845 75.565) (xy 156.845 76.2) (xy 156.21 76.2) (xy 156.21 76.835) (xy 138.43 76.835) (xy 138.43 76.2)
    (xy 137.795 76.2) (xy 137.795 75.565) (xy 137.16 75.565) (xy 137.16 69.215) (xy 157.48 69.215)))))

